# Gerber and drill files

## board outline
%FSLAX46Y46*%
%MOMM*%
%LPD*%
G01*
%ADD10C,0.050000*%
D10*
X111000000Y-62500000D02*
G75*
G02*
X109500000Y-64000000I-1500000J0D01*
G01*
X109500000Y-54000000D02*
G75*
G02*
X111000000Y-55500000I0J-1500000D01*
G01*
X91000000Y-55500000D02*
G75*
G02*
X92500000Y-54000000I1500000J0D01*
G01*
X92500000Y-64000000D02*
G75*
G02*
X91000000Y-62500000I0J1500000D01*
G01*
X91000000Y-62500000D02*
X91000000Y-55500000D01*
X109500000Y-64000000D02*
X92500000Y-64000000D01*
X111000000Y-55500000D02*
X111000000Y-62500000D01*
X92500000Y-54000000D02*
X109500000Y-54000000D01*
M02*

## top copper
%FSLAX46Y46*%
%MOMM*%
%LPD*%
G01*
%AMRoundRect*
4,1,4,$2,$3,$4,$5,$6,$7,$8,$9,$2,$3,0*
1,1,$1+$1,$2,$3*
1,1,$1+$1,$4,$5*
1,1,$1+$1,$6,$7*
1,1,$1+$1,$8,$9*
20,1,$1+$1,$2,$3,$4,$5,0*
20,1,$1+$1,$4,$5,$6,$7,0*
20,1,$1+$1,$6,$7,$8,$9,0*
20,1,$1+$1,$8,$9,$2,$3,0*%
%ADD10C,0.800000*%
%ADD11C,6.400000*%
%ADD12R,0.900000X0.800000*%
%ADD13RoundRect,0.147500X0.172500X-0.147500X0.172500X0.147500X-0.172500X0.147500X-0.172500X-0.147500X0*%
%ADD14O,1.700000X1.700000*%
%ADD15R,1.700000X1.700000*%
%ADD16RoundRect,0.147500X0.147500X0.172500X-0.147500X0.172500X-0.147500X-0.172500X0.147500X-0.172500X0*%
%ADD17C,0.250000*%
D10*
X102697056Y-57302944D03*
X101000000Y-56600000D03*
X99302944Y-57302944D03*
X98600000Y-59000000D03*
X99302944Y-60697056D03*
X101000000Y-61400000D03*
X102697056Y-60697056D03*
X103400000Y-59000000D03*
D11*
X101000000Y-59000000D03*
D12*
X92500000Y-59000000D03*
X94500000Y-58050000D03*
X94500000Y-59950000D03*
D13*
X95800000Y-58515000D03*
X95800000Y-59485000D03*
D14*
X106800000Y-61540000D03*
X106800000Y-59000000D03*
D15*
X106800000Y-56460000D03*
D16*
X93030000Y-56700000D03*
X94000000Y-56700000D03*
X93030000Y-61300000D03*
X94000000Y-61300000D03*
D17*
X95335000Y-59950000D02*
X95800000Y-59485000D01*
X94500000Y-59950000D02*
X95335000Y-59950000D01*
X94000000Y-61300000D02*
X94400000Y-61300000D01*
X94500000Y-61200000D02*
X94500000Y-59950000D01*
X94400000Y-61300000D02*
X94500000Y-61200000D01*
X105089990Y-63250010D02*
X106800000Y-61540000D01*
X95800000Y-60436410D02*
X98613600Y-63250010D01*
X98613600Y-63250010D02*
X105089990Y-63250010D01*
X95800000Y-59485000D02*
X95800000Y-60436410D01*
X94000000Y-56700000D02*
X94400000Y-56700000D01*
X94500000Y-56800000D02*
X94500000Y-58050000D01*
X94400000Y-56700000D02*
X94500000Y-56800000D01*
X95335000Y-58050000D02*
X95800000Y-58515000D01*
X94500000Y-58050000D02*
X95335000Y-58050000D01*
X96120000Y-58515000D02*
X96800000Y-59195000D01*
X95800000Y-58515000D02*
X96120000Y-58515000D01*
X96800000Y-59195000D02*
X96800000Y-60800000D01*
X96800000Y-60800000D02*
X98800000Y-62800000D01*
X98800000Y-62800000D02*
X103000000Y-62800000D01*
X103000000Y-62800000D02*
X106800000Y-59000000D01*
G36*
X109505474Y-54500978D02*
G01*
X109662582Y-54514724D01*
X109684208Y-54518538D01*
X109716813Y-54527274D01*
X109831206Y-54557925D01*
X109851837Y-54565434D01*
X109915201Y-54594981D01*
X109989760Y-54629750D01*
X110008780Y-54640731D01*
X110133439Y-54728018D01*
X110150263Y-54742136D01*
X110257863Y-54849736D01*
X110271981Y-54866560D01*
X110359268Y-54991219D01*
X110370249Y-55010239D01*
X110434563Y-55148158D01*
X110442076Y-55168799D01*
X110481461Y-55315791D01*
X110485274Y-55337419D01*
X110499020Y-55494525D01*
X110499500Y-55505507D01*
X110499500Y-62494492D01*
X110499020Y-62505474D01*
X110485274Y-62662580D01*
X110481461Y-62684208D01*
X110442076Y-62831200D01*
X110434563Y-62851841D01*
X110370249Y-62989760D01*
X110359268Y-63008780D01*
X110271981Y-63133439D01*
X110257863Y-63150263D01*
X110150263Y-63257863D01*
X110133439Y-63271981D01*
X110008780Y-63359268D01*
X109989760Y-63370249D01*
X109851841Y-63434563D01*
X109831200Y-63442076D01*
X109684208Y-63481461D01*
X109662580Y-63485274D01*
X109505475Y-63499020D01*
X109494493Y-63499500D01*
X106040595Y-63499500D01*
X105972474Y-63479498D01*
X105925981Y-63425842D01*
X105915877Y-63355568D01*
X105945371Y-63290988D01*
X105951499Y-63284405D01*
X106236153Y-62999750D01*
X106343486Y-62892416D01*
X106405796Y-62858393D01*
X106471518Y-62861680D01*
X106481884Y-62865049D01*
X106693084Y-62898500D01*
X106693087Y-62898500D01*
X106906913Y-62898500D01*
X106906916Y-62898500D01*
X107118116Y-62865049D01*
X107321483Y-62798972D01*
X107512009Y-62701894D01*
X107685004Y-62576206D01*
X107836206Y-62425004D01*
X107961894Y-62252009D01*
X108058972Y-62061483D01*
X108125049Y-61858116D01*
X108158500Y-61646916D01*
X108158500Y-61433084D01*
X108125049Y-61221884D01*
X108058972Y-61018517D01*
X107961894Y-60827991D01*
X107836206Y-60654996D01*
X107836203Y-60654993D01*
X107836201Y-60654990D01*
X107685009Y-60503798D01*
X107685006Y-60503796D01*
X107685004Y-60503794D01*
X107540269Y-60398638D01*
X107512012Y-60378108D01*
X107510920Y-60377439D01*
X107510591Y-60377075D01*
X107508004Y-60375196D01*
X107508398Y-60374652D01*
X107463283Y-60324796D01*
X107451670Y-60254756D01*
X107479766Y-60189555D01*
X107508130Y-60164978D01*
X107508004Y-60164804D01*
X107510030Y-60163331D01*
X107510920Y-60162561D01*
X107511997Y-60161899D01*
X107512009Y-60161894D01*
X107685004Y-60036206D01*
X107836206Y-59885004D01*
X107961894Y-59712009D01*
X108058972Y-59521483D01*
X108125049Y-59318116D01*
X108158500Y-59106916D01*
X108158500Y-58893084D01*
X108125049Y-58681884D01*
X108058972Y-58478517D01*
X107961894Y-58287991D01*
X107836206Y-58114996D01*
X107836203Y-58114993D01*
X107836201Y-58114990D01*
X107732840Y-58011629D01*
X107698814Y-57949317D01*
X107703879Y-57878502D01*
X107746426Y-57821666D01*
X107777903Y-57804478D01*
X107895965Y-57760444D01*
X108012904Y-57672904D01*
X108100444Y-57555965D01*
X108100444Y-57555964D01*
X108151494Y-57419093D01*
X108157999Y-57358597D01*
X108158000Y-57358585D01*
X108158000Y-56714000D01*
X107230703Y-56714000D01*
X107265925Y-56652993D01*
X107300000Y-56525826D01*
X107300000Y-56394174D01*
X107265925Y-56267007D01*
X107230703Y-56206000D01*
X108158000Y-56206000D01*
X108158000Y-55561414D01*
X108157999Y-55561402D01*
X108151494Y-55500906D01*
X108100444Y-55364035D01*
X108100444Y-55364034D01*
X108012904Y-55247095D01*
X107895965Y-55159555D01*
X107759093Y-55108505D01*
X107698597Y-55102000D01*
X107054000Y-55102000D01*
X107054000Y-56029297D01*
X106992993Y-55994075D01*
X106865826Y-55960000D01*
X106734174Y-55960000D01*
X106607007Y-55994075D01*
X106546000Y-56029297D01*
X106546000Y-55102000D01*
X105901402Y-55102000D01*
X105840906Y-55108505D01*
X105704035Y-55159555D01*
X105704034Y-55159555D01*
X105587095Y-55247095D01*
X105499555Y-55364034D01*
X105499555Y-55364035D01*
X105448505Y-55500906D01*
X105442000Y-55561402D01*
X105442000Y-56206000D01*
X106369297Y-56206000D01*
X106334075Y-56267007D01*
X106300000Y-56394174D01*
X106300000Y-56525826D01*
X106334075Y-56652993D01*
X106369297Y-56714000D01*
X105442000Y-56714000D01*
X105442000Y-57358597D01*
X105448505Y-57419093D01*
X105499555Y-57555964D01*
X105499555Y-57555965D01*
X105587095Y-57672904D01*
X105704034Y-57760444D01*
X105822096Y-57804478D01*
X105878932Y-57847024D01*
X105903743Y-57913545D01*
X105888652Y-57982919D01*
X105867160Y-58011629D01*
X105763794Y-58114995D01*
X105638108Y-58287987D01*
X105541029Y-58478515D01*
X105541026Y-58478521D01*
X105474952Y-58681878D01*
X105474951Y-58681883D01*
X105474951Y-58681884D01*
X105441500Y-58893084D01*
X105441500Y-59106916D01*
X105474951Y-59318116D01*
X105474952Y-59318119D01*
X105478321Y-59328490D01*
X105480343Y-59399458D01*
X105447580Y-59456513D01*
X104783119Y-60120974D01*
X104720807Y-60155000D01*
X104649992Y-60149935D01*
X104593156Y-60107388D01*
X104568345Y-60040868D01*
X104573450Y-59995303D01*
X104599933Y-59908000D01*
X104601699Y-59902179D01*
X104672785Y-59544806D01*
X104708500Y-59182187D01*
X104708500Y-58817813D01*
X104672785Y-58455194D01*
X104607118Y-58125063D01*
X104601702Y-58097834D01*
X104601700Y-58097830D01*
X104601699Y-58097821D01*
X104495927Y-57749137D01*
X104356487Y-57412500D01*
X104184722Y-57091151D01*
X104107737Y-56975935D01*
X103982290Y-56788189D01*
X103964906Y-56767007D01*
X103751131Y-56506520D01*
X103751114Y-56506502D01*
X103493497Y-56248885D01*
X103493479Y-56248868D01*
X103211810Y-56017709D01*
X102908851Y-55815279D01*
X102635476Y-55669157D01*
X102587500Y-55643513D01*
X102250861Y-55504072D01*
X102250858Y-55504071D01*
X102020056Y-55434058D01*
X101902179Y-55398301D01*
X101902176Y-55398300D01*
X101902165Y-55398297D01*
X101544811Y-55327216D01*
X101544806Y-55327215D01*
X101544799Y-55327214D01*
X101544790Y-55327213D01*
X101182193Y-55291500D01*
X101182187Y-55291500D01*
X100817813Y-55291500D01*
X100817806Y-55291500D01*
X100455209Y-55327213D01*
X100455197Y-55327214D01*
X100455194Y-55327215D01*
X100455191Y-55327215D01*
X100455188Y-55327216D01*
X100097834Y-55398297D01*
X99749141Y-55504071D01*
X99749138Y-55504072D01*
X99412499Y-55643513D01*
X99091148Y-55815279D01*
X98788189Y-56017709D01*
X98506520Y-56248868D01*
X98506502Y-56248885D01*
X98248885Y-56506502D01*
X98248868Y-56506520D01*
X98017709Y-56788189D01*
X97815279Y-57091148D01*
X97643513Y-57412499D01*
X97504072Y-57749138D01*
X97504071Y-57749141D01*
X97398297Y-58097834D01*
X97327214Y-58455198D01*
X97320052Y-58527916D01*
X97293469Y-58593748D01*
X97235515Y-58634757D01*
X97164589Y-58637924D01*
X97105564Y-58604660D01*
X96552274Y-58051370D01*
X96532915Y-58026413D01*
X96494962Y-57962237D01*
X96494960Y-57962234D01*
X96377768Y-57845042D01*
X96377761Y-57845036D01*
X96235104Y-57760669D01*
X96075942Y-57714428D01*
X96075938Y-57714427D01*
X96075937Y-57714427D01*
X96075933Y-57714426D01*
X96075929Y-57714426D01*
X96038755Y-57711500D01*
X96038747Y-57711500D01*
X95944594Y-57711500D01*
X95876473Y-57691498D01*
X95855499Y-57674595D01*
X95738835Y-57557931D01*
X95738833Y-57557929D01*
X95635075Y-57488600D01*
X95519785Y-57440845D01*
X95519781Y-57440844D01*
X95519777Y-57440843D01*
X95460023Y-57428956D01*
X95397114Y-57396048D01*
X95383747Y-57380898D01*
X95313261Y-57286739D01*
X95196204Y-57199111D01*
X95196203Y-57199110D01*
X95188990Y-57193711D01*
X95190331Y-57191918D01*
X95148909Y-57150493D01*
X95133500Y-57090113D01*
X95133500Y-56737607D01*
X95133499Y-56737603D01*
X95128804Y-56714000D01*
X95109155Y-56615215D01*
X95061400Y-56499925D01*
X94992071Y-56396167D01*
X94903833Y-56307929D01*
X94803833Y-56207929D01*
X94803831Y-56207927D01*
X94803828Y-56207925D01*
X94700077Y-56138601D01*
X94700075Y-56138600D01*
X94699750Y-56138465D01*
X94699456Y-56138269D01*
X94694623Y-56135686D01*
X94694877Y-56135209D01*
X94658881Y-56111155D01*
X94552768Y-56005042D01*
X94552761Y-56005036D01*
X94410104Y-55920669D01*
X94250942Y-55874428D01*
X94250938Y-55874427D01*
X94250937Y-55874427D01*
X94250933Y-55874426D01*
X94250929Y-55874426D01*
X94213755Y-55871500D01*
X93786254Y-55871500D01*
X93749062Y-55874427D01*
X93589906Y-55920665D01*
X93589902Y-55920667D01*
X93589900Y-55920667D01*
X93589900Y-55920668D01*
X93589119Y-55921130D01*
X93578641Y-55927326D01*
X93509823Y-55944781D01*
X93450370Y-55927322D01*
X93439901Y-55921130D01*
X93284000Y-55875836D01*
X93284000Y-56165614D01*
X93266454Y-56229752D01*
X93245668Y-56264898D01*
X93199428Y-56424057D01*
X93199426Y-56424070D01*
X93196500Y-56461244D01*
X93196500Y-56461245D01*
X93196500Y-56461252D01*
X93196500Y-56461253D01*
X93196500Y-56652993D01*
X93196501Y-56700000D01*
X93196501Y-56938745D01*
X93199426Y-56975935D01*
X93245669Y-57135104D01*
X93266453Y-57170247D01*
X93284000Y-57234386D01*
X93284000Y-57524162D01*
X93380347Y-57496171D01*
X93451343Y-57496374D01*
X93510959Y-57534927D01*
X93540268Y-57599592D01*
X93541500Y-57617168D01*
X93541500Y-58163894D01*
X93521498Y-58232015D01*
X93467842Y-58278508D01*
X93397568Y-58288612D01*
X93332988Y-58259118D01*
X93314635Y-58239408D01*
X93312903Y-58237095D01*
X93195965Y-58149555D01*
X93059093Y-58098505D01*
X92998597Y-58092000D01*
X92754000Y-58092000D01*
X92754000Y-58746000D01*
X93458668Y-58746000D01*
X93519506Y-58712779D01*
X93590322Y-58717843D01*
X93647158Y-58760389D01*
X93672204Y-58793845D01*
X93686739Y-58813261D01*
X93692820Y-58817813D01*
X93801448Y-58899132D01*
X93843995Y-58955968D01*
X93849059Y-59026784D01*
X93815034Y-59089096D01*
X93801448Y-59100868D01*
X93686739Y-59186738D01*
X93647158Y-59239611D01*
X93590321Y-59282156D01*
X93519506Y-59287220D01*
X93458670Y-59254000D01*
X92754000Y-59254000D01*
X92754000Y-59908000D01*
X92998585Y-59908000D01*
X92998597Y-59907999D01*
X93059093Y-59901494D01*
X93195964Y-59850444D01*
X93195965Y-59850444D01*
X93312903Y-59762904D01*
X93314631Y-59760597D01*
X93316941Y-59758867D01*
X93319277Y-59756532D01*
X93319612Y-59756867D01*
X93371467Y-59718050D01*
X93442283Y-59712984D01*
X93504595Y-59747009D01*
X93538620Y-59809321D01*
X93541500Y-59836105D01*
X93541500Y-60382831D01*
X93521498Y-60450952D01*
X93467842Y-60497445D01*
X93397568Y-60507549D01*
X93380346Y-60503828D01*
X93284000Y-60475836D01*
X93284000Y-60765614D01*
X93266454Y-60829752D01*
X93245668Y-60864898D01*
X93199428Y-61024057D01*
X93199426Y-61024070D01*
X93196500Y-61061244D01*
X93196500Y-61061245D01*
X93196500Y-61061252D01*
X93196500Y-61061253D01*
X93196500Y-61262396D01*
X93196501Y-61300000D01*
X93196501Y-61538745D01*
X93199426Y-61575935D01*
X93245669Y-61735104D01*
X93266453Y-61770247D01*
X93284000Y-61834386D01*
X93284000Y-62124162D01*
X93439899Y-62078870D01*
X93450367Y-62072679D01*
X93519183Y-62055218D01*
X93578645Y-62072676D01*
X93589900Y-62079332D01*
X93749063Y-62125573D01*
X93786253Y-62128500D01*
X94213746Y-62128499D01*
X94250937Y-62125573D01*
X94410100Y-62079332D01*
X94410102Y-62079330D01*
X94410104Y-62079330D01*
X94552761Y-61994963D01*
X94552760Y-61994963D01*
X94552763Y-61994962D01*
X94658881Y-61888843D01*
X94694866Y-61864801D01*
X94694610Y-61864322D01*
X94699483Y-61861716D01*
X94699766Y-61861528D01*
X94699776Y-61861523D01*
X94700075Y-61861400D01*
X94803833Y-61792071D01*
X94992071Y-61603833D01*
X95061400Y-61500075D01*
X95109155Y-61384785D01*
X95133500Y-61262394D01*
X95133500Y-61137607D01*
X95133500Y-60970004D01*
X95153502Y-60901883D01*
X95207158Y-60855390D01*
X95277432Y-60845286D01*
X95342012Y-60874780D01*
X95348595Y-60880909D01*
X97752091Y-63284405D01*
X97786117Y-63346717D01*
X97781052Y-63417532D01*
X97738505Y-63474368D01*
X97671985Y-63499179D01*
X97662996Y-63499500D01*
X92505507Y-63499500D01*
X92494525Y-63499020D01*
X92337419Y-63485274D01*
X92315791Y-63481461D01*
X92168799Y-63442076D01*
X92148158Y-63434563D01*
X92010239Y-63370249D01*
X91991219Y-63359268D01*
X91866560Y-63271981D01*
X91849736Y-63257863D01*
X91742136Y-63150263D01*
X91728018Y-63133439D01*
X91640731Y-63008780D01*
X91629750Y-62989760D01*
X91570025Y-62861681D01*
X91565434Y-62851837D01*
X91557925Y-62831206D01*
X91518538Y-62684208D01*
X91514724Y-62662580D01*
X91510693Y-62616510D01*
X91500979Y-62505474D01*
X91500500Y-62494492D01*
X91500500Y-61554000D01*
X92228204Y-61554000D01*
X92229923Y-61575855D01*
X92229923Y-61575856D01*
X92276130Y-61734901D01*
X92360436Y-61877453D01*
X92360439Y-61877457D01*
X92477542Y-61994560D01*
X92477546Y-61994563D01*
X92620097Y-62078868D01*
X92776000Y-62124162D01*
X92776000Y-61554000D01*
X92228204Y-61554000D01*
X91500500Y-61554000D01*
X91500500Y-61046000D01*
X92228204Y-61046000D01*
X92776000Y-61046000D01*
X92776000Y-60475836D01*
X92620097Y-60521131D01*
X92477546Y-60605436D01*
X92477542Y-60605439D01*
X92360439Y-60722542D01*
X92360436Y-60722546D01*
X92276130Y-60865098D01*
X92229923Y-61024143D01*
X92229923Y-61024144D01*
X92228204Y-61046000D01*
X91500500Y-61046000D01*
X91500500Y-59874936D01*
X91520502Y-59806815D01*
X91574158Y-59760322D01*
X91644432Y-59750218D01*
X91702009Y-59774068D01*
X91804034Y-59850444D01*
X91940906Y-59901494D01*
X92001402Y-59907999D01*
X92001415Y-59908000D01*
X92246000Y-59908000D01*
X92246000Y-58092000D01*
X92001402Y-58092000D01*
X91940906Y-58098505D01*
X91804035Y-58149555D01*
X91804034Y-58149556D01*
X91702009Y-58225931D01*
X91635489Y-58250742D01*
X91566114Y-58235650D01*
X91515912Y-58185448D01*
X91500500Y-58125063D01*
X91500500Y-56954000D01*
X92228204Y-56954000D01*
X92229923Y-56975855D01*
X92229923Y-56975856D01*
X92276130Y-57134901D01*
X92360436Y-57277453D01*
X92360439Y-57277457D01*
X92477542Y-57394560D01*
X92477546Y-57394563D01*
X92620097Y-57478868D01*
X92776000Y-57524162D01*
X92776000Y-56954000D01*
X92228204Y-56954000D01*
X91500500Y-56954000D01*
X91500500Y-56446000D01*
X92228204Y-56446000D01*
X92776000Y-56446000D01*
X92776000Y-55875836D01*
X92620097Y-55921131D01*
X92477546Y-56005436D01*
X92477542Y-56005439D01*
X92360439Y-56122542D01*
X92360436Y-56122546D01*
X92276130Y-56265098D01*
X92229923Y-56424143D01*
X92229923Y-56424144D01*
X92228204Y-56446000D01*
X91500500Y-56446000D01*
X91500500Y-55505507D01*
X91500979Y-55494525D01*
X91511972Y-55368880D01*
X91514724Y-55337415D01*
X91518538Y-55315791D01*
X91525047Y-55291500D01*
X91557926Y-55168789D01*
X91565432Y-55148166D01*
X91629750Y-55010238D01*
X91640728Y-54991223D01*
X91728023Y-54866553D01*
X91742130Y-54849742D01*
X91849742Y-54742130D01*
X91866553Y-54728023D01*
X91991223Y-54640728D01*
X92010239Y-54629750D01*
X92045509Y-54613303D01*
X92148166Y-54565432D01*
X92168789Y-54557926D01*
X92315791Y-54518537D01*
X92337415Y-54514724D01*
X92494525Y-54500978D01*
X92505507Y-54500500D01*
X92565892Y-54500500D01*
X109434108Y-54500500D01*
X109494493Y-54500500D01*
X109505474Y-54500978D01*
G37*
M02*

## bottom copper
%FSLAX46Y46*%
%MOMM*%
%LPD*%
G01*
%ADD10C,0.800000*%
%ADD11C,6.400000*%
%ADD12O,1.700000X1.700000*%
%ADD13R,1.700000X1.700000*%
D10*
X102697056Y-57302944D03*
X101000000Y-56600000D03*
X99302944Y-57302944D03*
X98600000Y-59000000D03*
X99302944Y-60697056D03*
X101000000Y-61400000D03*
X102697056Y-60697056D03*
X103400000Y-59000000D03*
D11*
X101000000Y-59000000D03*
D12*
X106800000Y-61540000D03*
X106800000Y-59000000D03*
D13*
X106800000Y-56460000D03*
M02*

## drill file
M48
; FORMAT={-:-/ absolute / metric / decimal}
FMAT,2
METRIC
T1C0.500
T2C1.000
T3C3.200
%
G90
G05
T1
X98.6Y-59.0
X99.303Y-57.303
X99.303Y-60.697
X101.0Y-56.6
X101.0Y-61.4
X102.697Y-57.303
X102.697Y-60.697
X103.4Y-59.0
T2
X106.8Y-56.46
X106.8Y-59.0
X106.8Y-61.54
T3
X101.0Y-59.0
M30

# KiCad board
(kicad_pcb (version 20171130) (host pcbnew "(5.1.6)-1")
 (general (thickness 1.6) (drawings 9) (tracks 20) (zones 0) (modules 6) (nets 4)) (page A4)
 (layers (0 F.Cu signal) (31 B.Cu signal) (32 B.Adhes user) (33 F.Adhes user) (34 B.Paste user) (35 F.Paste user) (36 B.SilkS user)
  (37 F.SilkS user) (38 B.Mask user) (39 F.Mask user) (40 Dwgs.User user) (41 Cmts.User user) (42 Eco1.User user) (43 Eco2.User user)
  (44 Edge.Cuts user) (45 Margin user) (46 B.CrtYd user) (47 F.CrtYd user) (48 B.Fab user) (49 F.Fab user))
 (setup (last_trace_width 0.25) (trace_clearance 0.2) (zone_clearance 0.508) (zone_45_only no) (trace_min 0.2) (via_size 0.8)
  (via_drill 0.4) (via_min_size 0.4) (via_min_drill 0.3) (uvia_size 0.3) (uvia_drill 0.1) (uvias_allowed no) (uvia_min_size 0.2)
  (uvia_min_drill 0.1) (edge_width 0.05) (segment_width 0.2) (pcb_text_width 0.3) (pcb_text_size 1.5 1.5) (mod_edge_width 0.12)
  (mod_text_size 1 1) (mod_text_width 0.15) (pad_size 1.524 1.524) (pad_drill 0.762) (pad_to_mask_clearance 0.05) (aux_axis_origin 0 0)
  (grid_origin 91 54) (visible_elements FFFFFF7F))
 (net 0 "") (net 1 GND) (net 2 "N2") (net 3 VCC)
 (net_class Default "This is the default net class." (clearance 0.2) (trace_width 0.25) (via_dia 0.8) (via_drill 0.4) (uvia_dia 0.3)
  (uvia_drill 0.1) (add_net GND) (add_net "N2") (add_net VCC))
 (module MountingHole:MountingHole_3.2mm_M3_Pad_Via (layer F.Cu) (at 101 59)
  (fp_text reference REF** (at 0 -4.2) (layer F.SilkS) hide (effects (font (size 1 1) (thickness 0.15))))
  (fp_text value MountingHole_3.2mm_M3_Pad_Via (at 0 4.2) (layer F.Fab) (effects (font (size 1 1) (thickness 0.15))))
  (pad 1 thru_hole circle (at 1.697056 -1.697056) (size 0.8 0.8) (drill 0.5) (layers *.Cu *.Mask))
  (pad 1 thru_hole circle (at 0 -2.4) (size 0.8 0.8) (drill 0.5) (layers *.Cu *.Mask))
  (pad 1 thru_hole circle (at -1.697056 -1.697056) (size 0.8 0.8) (drill 0.5) (layers *.Cu *.Mask))
  (pad 1 thru_hole circle (at -2.4 0) (size 0.8 0.8) (drill 0.5) (layers *.Cu *.Mask))
  (pad 1 thru_hole circle (at -1.697056 1.697056) (size 0.8 0.8) (drill 0.5) (layers *.Cu *.Mask))
  (pad 1 thru_hole circle (at 0 2.4) (size 0.8 0.8) (drill 0.5) (layers *.Cu *.Mask))
  (pad 1 thru_hole circle (at 1.697056 1.697056) (size 0.8 0.8) (drill 0.5) (layers *.Cu *.Mask))
  (pad 1 thru_hole circle (at 2.4 0) (size 0.8 0.8) (drill 0.5) (layers *.Cu *.Mask))
  (pad 1 thru_hole circle (at 0 0) (size 6.4 6.4) (drill 3.2) (layers *.Cu *.Mask)))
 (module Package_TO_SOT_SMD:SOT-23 (layer F.Cu) (at 93.5 59 180)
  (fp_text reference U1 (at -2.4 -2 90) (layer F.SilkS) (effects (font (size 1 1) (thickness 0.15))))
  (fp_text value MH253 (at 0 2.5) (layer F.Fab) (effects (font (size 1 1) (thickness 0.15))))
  (pad 3 smd rect (at 1 0 180) (size 0.9 0.8) (layers F.Cu F.Paste F.Mask) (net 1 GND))
  (pad 2 smd rect (at -1 0.95 180) (size 0.9 0.8) (layers F.Cu F.Paste F.Mask) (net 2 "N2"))
  (pad 1 smd rect (at -1 -0.95 180) (size 0.9 0.8) (layers F.Cu F.Paste F.Mask) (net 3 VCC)))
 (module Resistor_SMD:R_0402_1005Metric (layer F.Cu) (at 95.8 59 90)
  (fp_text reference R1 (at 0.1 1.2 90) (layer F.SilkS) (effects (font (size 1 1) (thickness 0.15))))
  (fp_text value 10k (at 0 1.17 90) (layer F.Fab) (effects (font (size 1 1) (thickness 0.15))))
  (pad 2 smd roundrect (at 0.485 0 90) (size 0.59 0.64) (layers F.Cu F.Paste F.Mask) (roundrect_rratio 0.25) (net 2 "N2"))
  (pad 1 smd roundrect (at -0.485 0 90) (size 0.59 0.64) (layers F.Cu F.Paste F.Mask) (roundrect_rratio 0.25) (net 3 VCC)))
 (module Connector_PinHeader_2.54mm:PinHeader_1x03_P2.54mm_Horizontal (layer F.Cu) (at 106.8 56.46)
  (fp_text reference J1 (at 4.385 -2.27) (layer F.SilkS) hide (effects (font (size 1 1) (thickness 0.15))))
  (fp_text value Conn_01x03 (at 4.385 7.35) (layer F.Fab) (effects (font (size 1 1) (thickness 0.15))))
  (pad 3 thru_hole oval (at 0 5.08) (size 1.7 1.7) (drill 1) (layers *.Cu *.Mask) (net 3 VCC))
  (pad 2 thru_hole oval (at 0 2.54) (size 1.7 1.7) (drill 1) (layers *.Cu *.Mask) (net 2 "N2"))
  (pad 1 thru_hole rect (at 0 0) (size 1.7 1.7) (drill 1) (layers *.Cu *.Mask) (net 1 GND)))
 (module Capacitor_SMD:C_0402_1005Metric (layer F.Cu) (at 93.515 56.7 180)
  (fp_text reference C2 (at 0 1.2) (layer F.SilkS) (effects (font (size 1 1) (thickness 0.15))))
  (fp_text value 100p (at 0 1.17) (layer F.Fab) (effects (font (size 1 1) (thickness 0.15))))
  (pad 2 smd roundrect (at 0.485 0 180) (size 0.59 0.64) (layers F.Cu F.Paste F.Mask) (roundrect_rratio 0.25) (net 1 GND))
  (pad 1 smd roundrect (at -0.485 0 180) (size 0.59 0.64) (layers F.Cu F.Paste F.Mask) (roundrect_rratio 0.25) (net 2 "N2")))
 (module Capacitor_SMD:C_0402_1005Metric (layer F.Cu) (at 93.515 61.3 180)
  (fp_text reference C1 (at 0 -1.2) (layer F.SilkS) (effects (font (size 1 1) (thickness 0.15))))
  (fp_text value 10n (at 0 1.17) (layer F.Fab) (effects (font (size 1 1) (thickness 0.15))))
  (pad 2 smd roundrect (at 0.485 0 180) (size 0.59 0.64) (layers F.Cu F.Paste F.Mask) (roundrect_rratio 0.25) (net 1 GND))
  (pad 1 smd roundrect (at -0.485 0 180) (size 0.59 0.64) (layers F.Cu F.Paste F.Mask) (roundrect_rratio 0.25) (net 3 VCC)))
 (gr_arc (start 109.5 62.5) (end 109.5 64) (angle -90) (layer Edge.Cuts) (width 0.05))
 (gr_arc (start 109.5 55.5) (end 111 55.5) (angle -90) (layer Edge.Cuts) (width 0.05))
 (gr_arc (start 92.5 55.5) (end 92.5 54) (angle -90) (layer Edge.Cuts) (width 0.05))
 (gr_arc (start 92.5 62.5) (end 91 62.5) (angle -90) (layer Edge.Cuts) (width 0.05))
 (gr_line (start 91 62.5) (end 91 55.5) (layer Edge.Cuts) (width 0.05))
 (gr_line (start 109.5 64) (end 92.5 64) (layer Edge.Cuts) (width 0.05))
 (gr_line (start 111 55.5) (end 111 62.5) (layer Edge.Cuts) (width 0.05))
 (gr_line (start 92.5 54) (end 109.5 54) (layer Edge.Cuts) (width 0.05))
 (segment (start 95.335 59.95) (end 95.8 59.485) (width 0.25) (layer F.Cu) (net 3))
 (segment (start 94.5 59.95) (end 95.335 59.95) (width 0.25) (layer F.Cu) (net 3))
 (segment (start 94 61.3) (end 94.4 61.3) (width 0.25) (layer F.Cu) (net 3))
 (segment (start 94.5 61.2) (end 94.5 59.95) (width 0.25) (layer F.Cu) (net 3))
 (segment (start 94.4 61.3) (end 94.5 61.2) (width 0.25) (layer F.Cu) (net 3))
 (segment (start 105.08999 63.25001) (end 106.8 61.54) (width 0.25) (layer F.Cu) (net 3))
 (segment (start 95.8 60.43641) (end 98.6136 63.25001) (width 0.25) (layer F.Cu) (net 3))
 (segment (start 98.6136 63.25001) (end 105.08999 63.25001) (width 0.25) (layer F.Cu) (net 3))
 (segment (start 95.8 59.485) (end 95.8 60.43641) (width 0.25) (layer F.Cu) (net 3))
 (segment (start 94 56.7) (end 94.4 56.7) (width 0.25) (layer F.Cu) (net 2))
 (segment (start 94.5 56.8) (end 94.5 58.05) (width 0.25) (layer F.Cu) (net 2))
 (segment (start 94.4 56.7) (end 94.5 56.8) (width 0.25) (layer F.Cu) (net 2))
 (segment (start 95.335 58.05) (end 95.8 58.515) (width 0.25) (layer F.Cu) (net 2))
 (segment (start 94.5 58.05) (end 95.335 58.05) (width 0.25) (layer F.Cu) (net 2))
 (segment (start 96.12 58.515) (end 96.8 59.195) (width 0.25) (layer F.Cu) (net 2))
 (segment (start 95.8 58.515) (end 96.12 58.515) (width 0.25) (layer F.Cu) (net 2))
 (segment (start 96.8 59.195) (end 96.8 60.8) (width 0.25) (layer F.Cu) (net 2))
 (segment (start 96.8 60.8) (end 98.8 62.8) (width 0.25) (layer F.Cu) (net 2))
 (segment (start 98.8 62.8) (end 103 62.8) (width 0.25) (layer F.Cu) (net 2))
 (segment (start 103 62.8) (end 106.8 59) (width 0.25) (layer F.Cu) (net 2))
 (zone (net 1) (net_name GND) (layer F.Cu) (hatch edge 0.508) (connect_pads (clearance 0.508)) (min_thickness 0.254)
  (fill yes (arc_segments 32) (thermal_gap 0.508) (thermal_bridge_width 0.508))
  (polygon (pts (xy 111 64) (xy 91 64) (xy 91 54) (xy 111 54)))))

